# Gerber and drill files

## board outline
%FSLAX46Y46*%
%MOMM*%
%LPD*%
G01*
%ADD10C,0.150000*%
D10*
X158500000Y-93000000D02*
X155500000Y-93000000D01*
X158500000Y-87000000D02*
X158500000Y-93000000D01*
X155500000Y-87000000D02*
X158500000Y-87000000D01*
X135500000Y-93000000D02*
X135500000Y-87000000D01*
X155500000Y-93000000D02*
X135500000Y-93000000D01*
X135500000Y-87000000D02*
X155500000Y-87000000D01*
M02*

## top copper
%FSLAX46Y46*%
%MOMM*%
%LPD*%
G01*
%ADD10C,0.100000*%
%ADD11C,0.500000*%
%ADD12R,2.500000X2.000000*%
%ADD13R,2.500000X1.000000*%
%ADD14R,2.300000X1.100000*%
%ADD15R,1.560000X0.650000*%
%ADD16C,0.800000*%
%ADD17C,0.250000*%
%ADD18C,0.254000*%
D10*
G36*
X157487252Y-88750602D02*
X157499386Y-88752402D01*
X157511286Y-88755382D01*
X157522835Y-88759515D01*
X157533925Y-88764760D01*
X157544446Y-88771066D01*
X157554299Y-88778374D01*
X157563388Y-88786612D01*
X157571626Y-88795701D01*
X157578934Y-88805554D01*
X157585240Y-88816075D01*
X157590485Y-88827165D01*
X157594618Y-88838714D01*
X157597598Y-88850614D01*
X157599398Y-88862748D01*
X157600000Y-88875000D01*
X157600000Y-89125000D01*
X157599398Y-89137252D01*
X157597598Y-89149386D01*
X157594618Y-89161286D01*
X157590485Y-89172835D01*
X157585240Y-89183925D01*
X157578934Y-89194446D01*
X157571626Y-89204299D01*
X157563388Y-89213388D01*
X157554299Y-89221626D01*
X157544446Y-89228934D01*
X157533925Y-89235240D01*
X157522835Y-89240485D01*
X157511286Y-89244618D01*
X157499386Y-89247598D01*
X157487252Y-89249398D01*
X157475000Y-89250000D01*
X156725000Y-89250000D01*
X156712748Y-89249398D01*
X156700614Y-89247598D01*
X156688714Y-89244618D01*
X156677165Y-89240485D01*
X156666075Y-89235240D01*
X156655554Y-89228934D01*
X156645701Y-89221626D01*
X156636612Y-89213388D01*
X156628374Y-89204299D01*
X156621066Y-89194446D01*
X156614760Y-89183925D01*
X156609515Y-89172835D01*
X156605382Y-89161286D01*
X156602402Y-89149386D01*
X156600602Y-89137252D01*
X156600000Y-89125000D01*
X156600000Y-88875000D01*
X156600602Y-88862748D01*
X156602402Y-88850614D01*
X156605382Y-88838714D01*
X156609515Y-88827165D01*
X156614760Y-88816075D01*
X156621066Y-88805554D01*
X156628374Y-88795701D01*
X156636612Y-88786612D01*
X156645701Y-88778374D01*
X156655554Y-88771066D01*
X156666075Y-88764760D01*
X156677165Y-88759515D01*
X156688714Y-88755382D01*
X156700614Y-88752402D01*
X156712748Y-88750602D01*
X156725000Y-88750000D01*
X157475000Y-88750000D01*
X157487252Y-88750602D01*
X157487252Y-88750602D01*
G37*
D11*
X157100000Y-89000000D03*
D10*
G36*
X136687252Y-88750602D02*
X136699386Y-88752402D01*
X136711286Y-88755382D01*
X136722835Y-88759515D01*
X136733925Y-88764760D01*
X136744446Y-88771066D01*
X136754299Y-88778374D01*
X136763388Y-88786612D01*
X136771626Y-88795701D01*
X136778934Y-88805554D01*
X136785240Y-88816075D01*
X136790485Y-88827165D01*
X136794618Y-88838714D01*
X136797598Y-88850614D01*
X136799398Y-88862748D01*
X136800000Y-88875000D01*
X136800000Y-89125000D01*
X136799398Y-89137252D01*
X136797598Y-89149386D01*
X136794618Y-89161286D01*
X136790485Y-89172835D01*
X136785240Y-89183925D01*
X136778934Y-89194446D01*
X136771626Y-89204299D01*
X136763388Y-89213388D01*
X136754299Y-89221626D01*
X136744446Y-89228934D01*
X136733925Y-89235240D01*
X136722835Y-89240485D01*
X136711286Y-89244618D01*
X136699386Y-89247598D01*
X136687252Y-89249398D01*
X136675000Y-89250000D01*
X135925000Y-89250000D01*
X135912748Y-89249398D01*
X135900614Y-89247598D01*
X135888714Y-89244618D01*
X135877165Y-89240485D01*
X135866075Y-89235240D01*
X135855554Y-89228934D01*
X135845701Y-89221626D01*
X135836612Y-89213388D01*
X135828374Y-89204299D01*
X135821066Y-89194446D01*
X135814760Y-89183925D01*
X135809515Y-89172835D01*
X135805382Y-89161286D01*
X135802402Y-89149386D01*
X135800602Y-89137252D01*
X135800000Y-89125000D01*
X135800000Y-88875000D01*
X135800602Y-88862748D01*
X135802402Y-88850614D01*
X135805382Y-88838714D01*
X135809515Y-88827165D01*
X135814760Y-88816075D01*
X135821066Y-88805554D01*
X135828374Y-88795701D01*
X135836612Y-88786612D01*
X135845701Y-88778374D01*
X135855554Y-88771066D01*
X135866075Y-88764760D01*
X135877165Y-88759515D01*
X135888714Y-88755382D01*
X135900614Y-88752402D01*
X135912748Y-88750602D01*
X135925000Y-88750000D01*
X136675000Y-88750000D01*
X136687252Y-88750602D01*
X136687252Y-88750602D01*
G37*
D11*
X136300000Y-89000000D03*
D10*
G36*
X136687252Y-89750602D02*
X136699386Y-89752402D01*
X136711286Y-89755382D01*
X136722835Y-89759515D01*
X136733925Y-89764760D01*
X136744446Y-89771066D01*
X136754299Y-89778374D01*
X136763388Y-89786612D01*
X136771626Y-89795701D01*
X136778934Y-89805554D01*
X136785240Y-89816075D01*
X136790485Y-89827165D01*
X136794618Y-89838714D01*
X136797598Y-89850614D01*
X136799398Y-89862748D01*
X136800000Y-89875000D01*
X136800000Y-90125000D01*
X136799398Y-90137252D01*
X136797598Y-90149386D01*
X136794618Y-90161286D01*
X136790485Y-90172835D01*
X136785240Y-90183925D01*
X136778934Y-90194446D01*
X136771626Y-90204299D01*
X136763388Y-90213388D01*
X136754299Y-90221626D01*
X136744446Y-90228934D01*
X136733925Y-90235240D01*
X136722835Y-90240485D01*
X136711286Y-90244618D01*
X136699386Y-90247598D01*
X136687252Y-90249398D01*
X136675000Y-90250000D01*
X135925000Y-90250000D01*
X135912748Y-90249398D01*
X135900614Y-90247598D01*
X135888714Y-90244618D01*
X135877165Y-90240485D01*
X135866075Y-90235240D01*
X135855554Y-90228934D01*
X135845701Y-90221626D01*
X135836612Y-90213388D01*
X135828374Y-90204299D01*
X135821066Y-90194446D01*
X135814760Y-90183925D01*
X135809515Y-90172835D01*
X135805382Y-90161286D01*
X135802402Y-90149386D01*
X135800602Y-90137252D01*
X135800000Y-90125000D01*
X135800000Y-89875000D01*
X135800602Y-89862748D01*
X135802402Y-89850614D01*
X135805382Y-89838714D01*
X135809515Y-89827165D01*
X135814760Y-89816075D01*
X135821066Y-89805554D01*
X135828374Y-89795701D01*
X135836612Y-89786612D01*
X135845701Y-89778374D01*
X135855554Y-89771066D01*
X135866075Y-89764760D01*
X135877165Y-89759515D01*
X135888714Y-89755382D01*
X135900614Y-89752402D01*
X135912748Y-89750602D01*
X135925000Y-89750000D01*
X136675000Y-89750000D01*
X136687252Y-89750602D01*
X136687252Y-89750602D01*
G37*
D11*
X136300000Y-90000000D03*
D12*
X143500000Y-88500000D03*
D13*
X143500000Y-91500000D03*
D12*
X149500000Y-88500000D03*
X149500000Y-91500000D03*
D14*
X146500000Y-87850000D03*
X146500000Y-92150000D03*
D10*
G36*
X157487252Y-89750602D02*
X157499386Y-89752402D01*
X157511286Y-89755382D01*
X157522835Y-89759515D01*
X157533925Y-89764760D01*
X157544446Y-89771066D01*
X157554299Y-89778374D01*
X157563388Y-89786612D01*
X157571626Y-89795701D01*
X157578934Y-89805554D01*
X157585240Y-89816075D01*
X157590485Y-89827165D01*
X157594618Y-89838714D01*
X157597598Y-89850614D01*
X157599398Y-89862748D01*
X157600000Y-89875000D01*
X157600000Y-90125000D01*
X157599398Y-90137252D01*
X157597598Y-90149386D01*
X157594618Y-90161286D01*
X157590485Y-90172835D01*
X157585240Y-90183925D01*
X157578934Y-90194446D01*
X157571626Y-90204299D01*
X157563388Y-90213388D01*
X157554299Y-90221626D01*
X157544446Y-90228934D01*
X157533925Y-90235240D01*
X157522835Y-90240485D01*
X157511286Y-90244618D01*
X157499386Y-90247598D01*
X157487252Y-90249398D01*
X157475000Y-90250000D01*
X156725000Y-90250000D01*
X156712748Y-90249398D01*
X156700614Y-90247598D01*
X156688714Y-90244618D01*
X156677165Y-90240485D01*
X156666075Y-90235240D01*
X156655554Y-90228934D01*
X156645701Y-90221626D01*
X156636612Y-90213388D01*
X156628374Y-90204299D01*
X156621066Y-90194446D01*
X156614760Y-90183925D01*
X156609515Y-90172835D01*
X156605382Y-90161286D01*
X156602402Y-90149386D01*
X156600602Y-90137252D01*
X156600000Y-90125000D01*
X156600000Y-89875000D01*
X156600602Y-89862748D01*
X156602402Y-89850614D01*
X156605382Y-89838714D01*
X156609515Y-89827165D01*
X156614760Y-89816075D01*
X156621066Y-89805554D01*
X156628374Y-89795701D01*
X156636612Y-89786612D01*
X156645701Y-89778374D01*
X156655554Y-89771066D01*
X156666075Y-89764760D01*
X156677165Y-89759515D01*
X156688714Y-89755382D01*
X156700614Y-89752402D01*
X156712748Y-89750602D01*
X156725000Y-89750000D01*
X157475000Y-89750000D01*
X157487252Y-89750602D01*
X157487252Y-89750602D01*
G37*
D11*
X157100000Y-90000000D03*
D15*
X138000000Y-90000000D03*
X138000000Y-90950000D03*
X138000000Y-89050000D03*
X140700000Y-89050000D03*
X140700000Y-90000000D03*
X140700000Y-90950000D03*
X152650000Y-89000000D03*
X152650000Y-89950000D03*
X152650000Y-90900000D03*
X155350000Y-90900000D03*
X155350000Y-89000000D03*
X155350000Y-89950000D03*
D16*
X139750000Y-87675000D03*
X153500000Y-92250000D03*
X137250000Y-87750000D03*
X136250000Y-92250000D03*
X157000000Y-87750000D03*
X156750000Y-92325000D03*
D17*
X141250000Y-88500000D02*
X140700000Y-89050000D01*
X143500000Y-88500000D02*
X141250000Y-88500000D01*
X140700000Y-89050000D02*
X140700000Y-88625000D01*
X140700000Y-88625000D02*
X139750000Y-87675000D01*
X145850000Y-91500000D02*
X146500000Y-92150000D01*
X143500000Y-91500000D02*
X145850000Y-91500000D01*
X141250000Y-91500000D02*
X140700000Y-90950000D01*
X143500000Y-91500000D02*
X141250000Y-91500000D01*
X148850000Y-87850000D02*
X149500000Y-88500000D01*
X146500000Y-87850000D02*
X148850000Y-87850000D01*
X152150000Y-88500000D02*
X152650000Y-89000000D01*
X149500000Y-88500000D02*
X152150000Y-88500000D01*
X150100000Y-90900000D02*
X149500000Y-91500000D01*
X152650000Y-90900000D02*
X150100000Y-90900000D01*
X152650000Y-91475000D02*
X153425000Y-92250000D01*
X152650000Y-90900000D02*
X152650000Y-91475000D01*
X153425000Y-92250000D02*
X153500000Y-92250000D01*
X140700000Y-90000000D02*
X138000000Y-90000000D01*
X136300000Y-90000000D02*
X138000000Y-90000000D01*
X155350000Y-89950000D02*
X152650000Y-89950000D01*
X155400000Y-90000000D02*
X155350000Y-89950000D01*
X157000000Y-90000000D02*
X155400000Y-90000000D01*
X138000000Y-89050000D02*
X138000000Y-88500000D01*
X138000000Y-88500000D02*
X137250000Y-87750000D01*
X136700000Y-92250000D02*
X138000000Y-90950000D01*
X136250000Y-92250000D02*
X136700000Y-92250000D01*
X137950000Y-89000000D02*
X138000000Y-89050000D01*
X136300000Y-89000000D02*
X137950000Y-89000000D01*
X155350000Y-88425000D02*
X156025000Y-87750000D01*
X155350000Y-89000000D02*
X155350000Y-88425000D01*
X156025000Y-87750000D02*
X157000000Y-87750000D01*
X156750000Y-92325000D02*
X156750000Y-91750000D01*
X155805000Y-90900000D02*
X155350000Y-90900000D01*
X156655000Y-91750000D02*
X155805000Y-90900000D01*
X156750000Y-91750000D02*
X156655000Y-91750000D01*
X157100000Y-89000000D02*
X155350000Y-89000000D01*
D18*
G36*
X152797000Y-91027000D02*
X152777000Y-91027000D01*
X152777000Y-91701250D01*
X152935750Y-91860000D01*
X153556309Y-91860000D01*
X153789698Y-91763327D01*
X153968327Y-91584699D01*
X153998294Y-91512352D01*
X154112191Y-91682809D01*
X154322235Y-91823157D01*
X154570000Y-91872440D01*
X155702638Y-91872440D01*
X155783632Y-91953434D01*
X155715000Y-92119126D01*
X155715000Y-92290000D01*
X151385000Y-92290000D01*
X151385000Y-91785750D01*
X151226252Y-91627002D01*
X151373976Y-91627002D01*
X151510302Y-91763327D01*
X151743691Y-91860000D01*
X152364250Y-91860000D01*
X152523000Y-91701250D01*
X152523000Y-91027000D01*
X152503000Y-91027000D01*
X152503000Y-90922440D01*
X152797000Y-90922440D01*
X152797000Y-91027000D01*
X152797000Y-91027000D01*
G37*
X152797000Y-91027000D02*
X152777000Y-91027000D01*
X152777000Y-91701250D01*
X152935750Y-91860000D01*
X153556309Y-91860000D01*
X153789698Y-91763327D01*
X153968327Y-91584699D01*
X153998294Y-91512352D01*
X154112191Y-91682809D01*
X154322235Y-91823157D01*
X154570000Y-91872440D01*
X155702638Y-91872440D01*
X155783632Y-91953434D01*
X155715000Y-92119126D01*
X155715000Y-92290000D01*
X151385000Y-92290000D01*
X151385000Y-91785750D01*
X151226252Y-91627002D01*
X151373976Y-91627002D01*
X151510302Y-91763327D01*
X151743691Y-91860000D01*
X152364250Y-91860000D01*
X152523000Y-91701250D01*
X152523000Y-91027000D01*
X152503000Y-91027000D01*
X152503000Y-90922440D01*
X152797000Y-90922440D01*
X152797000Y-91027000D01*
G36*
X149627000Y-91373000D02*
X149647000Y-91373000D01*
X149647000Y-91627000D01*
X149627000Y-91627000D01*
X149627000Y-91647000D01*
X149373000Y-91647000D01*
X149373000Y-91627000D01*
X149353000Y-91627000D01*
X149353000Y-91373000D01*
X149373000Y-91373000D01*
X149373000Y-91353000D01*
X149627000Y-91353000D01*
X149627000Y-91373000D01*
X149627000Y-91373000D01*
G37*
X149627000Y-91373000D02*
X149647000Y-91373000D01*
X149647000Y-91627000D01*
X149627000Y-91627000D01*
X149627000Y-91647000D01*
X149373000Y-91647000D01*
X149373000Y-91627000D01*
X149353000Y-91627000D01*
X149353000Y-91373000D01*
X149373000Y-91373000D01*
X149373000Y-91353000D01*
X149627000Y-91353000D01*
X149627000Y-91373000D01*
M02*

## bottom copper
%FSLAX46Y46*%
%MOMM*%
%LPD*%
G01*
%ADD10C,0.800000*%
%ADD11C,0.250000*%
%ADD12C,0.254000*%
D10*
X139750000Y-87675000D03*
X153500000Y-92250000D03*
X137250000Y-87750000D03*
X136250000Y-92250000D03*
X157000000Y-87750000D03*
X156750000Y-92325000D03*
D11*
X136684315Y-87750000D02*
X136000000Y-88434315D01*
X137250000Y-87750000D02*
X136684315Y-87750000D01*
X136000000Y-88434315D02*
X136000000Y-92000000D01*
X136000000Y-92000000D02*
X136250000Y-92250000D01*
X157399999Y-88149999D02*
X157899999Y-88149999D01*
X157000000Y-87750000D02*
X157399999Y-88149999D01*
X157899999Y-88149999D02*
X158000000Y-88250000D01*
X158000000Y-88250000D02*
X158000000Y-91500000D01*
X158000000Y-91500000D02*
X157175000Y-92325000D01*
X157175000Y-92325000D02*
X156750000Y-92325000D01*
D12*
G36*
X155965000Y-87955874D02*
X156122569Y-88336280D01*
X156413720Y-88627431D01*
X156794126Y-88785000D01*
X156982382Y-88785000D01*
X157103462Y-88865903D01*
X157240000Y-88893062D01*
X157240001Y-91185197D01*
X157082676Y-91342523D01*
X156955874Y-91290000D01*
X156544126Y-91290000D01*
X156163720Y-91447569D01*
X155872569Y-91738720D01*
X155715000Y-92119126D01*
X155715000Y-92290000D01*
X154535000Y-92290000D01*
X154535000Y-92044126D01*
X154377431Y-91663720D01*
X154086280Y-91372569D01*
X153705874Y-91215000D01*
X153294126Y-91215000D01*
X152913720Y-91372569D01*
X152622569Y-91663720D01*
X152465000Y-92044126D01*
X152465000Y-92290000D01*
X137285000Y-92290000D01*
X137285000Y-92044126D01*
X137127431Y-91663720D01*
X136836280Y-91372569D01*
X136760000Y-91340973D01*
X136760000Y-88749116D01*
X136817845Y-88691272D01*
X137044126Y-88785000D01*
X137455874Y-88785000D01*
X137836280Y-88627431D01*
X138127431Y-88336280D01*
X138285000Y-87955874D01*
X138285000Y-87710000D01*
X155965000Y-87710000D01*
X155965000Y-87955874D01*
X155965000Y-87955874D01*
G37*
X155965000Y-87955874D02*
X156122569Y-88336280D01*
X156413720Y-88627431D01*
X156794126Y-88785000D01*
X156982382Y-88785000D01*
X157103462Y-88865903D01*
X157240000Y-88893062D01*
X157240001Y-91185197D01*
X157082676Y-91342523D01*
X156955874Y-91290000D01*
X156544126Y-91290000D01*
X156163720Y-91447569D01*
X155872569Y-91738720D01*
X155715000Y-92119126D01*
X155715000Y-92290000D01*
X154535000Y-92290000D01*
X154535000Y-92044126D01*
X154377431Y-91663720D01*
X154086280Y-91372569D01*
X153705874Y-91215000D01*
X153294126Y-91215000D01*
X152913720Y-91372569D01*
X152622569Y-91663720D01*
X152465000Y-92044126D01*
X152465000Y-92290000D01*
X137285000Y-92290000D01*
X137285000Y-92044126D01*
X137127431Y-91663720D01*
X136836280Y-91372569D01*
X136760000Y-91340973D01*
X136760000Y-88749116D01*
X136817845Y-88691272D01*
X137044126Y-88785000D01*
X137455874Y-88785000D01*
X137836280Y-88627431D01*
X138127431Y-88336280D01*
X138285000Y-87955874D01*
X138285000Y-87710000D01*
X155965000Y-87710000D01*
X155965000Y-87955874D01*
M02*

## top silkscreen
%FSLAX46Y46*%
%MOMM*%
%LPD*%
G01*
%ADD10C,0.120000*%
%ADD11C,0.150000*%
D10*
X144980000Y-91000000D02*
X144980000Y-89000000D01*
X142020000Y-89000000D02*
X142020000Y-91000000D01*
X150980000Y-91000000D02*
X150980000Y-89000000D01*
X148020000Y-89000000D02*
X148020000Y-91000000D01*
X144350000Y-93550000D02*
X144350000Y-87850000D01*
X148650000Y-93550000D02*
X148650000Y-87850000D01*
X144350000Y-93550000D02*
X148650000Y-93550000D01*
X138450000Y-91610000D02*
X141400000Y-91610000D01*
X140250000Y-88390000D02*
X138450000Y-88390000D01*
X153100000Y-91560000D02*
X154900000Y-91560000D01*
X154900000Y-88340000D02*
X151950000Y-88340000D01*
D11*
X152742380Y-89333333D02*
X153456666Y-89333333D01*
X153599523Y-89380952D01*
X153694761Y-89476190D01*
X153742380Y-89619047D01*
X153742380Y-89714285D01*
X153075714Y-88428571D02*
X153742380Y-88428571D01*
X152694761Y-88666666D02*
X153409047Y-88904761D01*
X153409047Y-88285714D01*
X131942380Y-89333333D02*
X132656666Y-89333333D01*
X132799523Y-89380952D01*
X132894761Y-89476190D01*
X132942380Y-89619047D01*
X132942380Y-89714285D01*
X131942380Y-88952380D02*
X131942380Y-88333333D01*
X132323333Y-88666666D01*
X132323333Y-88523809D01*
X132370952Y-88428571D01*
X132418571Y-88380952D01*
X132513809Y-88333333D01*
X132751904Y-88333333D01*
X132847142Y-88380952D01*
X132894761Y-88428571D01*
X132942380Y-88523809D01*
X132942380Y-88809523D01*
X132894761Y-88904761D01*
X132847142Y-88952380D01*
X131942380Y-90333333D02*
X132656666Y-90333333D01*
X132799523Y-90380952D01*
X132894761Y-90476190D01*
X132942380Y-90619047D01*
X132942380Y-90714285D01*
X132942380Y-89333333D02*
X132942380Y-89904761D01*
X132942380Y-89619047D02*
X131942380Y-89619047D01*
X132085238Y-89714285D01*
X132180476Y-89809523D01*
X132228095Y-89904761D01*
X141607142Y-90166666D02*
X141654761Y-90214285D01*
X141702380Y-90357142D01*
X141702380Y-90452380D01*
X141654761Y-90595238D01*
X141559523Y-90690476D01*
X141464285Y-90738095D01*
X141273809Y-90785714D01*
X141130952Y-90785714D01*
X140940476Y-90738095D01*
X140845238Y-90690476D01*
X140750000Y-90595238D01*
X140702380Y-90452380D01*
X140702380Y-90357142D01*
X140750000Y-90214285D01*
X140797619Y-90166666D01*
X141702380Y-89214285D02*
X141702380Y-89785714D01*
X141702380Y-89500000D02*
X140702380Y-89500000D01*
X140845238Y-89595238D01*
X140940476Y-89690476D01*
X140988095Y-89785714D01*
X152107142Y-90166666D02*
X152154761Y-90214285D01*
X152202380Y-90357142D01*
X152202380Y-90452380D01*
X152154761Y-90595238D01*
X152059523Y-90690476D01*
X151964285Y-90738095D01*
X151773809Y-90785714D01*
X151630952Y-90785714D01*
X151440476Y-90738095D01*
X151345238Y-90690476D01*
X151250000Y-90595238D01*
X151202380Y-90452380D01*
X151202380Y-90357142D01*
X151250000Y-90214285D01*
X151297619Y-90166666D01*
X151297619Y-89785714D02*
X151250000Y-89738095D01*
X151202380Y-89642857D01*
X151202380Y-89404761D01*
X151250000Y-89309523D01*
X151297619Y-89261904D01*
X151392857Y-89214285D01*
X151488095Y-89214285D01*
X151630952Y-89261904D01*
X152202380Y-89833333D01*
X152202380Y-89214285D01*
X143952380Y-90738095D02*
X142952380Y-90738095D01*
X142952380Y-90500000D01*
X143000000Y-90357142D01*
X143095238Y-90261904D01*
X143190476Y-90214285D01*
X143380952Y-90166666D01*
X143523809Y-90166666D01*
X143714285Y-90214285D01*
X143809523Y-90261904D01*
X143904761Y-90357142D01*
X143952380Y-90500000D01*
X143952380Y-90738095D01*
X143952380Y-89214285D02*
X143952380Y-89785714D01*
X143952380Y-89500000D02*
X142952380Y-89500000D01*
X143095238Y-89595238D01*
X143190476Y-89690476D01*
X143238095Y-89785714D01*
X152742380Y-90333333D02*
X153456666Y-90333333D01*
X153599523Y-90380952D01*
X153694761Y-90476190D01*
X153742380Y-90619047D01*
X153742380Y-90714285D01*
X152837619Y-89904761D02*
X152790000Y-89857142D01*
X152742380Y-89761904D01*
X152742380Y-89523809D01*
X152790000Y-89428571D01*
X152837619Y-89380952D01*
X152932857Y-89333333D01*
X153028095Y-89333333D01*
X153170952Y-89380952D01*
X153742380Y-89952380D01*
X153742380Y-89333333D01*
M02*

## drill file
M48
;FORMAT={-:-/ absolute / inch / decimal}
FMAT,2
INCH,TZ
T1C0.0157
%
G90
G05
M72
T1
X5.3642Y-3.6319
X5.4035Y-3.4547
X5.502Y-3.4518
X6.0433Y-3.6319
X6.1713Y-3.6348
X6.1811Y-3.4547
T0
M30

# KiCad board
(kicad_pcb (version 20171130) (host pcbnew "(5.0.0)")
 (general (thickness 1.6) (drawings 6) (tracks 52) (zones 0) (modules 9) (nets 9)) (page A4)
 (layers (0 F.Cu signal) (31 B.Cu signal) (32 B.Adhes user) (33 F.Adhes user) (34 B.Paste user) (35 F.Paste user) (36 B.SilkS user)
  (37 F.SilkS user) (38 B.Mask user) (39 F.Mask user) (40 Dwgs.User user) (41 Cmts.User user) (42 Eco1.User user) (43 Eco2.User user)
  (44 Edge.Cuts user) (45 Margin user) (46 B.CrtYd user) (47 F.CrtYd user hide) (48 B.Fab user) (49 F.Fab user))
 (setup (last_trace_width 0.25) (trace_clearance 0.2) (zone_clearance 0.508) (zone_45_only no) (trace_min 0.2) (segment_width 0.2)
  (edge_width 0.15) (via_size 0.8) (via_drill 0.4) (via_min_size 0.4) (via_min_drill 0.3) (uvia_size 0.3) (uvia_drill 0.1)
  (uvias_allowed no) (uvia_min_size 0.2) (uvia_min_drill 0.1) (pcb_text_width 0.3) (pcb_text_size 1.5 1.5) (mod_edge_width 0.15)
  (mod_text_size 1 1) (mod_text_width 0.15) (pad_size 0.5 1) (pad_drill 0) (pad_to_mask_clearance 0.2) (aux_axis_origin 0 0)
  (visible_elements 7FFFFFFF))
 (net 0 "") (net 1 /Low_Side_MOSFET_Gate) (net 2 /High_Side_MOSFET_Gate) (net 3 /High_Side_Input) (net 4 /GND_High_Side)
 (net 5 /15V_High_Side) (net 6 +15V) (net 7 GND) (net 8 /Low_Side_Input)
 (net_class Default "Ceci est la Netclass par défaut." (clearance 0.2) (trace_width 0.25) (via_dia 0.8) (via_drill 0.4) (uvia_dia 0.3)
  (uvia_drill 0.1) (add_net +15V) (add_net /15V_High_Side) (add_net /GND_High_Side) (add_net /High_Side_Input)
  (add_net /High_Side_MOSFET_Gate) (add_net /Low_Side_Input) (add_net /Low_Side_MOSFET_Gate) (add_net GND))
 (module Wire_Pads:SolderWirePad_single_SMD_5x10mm (layer F.Cu) (at 157.1 89 90)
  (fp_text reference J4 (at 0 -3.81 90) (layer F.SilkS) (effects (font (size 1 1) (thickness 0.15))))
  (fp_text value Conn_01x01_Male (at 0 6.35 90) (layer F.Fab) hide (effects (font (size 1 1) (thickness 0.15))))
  (pad 1 smd roundrect (at 0 0 90) (size 0.5 1) (layers F.Cu F.Paste F.Mask) (roundrect_rratio 0.25) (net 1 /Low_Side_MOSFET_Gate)))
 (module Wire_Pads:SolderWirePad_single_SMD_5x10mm (layer F.Cu) (at 136.3 89 90)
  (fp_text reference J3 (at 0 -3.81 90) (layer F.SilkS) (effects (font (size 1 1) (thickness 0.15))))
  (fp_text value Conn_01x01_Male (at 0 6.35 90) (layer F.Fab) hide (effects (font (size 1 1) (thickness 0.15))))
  (pad 1 smd roundrect (at 0 0 90) (size 0.5 1) (layers F.Cu F.Paste F.Mask) (roundrect_rratio 0.25) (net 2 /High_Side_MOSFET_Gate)))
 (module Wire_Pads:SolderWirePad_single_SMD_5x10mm (layer F.Cu) (at 136.3 90 90)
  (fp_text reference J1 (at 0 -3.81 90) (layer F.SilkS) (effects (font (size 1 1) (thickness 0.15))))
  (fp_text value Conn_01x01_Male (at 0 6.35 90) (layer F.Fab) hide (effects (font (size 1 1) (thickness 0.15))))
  (pad 1 smd roundrect (at 0 0 90) (size 0.5 1) (layers F.Cu F.Paste F.Mask) (roundrect_rratio 0.25) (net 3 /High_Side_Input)))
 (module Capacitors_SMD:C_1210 (layer F.Cu) (at 143.5 90 90)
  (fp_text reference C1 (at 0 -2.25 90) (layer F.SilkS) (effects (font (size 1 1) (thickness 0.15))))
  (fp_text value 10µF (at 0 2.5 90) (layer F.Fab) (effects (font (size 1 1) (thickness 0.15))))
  (fp_line (start -1 1.48) (end 1 1.48) (layer F.SilkS) (width 0.12))
  (fp_line (start 1 -1.48) (end -1 -1.48) (layer F.SilkS) (width 0.12))
  (pad 2 smd rect (at 1.5 0 90) (size 2 2.5) (layers F.Cu F.Paste F.Mask) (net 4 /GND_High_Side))
  (pad 1 smd rect (at -1.5 0 90) (size 1 2.5) (layers F.Cu F.Paste F.Mask) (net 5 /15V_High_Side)))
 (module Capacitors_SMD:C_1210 (layer F.Cu) (at 149.5 90 270)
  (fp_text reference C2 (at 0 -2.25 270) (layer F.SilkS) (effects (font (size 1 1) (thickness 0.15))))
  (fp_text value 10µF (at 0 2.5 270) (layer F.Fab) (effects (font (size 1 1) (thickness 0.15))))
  (fp_line (start 1 -1.48) (end -1 -1.48) (layer F.SilkS) (width 0.12))
  (fp_line (start -1 1.48) (end 1 1.48) (layer F.SilkS) (width 0.12))
  (pad 1 smd rect (at -1.5 0 270) (size 2 2.5) (layers F.Cu F.Paste F.Mask) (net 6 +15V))
  (pad 2 smd rect (at 1.5 0 270) (size 2 2.5) (layers F.Cu F.Paste F.Mask) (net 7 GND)))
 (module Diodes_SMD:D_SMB (layer F.Cu) (at 146.5 90 90)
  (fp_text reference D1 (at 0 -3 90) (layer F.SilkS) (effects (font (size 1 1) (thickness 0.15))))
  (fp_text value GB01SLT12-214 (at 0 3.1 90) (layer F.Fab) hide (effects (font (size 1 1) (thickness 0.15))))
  (fp_line (start -3.55 -2.15) (end 2.15 -2.15) (layer F.SilkS) (width 0.12))
  (fp_line (start -3.55 2.15) (end 2.15 2.15) (layer F.SilkS) (width 0.12))
  (fp_line (start -3.55 -2.15) (end -3.55 2.15) (layer F.SilkS) (width 0.12))
  (pad 2 smd rect (at 2.15 0 90) (size 1.1 2.3) (layers F.Cu F.Paste F.Mask) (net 6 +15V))
  (pad 1 smd rect (at -2.15 0 90) (size 1.1 2.3) (layers F.Cu F.Paste F.Mask) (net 5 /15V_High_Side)))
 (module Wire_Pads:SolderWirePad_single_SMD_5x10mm (layer F.Cu) (at 157.1 90 90)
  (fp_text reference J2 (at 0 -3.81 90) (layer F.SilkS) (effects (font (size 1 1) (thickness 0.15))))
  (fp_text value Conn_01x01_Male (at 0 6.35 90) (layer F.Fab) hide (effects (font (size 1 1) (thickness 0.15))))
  (pad 1 smd roundrect (at 0 0 90) (size 0.5 1) (layers F.Cu F.Paste F.Mask) (roundrect_rratio 0.25) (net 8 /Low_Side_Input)
   (zone_connect 0)))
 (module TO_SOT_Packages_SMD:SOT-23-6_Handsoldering (layer F.Cu) (at 139.35 90 180)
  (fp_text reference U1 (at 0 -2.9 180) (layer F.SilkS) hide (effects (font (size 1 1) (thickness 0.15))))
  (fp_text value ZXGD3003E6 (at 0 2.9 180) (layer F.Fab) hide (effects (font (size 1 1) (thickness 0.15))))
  (fp_line (start 0.9 -1.61) (end -2.05 -1.61) (layer F.SilkS) (width 0.12))
  (fp_line (start -0.9 1.61) (end 0.9 1.61) (layer F.SilkS) (width 0.12))
  (pad 5 smd rect (at 1.35 0 180) (size 1.56 0.65) (layers F.Cu F.Paste F.Mask) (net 3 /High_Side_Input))
  (pad 6 smd rect (at 1.35 -0.95 180) (size 1.56 0.65) (layers F.Cu F.Paste F.Mask) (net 2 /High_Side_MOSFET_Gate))
  (pad 4 smd rect (at 1.35 0.95 180) (size 1.56 0.65) (layers F.Cu F.Paste F.Mask) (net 2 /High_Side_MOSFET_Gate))
  (pad 3 smd rect (at -1.35 0.95 180) (size 1.56 0.65) (layers F.Cu F.Paste F.Mask) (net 4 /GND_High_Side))
  (pad 2 smd rect (at -1.35 0 180) (size 1.56 0.65) (layers F.Cu F.Paste F.Mask) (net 3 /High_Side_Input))
  (pad 1 smd rect (at -1.35 -0.95 180) (size 1.56 0.65) (layers F.Cu F.Paste F.Mask) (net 5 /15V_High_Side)))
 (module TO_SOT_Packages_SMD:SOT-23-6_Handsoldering (layer F.Cu) (at 154 89.95)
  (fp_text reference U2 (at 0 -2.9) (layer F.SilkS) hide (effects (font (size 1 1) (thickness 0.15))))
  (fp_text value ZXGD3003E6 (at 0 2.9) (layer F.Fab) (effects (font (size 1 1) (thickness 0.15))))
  (fp_line (start -0.9 1.61) (end 0.9 1.61) (layer F.SilkS) (width 0.12))
  (fp_line (start 0.9 -1.61) (end -2.05 -1.61) (layer F.SilkS) (width 0.12))
  (pad 1 smd rect (at -1.35 -0.95) (size 1.56 0.65) (layers F.Cu F.Paste F.Mask) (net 6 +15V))
  (pad 2 smd rect (at -1.35 0) (size 1.56 0.65) (layers F.Cu F.Paste F.Mask) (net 8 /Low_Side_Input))
  (pad 3 smd rect (at -1.35 0.95) (size 1.56 0.65) (layers F.Cu F.Paste F.Mask) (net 7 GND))
  (pad 4 smd rect (at 1.35 0.95) (size 1.56 0.65) (layers F.Cu F.Paste F.Mask) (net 1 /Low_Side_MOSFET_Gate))
  (pad 6 smd rect (at 1.35 -0.95) (size 1.56 0.65) (layers F.Cu F.Paste F.Mask) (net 1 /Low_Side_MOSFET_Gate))
  (pad 5 smd rect (at 1.35 0) (size 1.56 0.65) (layers F.Cu F.Paste F.Mask) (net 8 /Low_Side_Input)))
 (gr_line (start 158.5 93) (end 155.5 93) (layer Edge.Cuts) (width 0.15))
 (gr_line (start 158.5 87) (end 158.5 93) (layer Edge.Cuts) (width 0.15))
 (gr_line (start 155.5 87) (end 158.5 87) (layer Edge.Cuts) (width 0.15))
 (gr_line (start 135.5 93) (end 135.5 87) (layer Edge.Cuts) (width 0.15))
 (gr_line (start 155.5 93) (end 135.5 93) (layer Edge.Cuts) (width 0.15))
 (gr_line (start 135.5 87) (end 155.5 87) (layer Edge.Cuts) (width 0.15))
 (segment (start 141.25 88.5) (end 140.7 89.05) (width 0.25) (layer F.Cu) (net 4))
 (segment (start 143.5 88.5) (end 141.25 88.5) (width 0.25) (layer F.Cu) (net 4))
 (via (at 139.75 87.675) (size 0.8) (drill 0.4) (layers F.Cu B.Cu) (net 4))
 (segment (start 140.7 89.05) (end 140.7 88.625) (width 0.25) (layer F.Cu) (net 4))
 (segment (start 140.7 88.625) (end 139.75 87.675) (width 0.25) (layer F.Cu) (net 4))
 (segment (start 145.85 91.5) (end 146.5 92.15) (width 0.25) (layer F.Cu) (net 5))
 (segment (start 143.5 91.5) (end 145.85 91.5) (width 0.25) (layer F.Cu) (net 5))
 (segment (start 141.25 91.5) (end 140.7 90.95) (width 0.25) (layer F.Cu) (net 5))
 (segment (start 143.5 91.5) (end 141.25 91.5) (width 0.25) (layer F.Cu) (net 5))
 (segment (start 148.85 87.85) (end 149.5 88.5) (width 0.25) (layer F.Cu) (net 6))
 (segment (start 146.5 87.85) (end 148.85 87.85) (width 0.25) (layer F.Cu) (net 6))
 (segment (start 152.15 88.5) (end 152.65 89) (width 0.25) (layer F.Cu) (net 6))
 (segment (start 149.5 88.5) (end 152.15 88.5) (width 0.25) (layer F.Cu) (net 6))
 (segment (start 150.1 90.9) (end 149.5 91.5) (width 0.25) (layer F.Cu) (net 7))
 (segment (start 152.65 90.9) (end 150.1 90.9) (width 0.25) (layer F.Cu) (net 7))
 (segment (start 152.65 91.475) (end 153.425 92.25) (width 0.25) (layer F.Cu) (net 7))
 (segment (start 152.65 90.9) (end 152.65 91.475) (width 0.25) (layer F.Cu) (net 7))
 (via (at 153.5 92.25) (size 0.8) (drill 0.4) (layers F.Cu B.Cu) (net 7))
 (segment (start 153.425 92.25) (end 153.5 92.25) (width 0.25) (layer F.Cu) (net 7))
 (segment (start 140.7 90) (end 138 90) (width 0.25) (layer F.Cu) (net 3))
 (segment (start 136.3 90) (end 138 90) (width 0.25) (layer F.Cu) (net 3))
 (segment (start 155.35 89.95) (end 152.65 89.95) (width 0.25) (layer F.Cu) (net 8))
 (segment (start 155.4 90) (end 155.35 89.95) (width 0.25) (layer F.Cu) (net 8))
 (segment (start 157 90) (end 155.4 90) (width 0.25) (layer F.Cu) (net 8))
 (via (at 137.25 87.75) (size 0.8) (drill 0.4) (layers F.Cu B.Cu) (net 2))
 (segment (start 138 89.05) (end 138 88.5) (width 0.25) (layer F.Cu) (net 2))
 (segment (start 138 88.5) (end 137.25 87.75) (width 0.25) (layer F.Cu) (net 2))
 (segment (start 136.684315 87.75) (end 136 88.434315) (width 0.25) (layer B.Cu) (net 2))
 (segment (start 137.25 87.75) (end 136.684315 87.75) (width 0.25) (layer B.Cu) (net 2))
 (via (at 136.25 92.25) (size 0.8) (drill 0.4) (layers F.Cu B.Cu) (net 2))
 (segment (start 136 88.434315) (end 136 92) (width 0.25) (layer B.Cu) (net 2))
 (segment (start 136 92) (end 136.25 92.25) (width 0.25) (layer B.Cu) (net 2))
 (segment (start 136.7 92.25) (end 138 90.95) (width 0.25) (layer F.Cu) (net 2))
 (segment (start 136.25 92.25) (end 136.7 92.25) (width 0.25) (layer F.Cu) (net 2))
 (segment (start 137.95 89) (end 138 89.05) (width 0.25) (layer F.Cu) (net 2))
 (segment (start 136.3 89) (end 137.95 89) (width 0.25) (layer F.Cu) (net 2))
 (segment (start 155.35 88.425) (end 156.025 87.75) (width 0.25) (layer F.Cu) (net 1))
 (segment (start 155.35 89) (end 155.35 88.425) (width 0.25) (layer F.Cu) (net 1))
 (via (at 157 87.75) (size 0.8) (drill 0.4) (layers F.Cu B.Cu) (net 1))
 (segment (start 156.025 87.75) (end 157 87.75) (width 0.25) (layer F.Cu) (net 1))
 (segment (start 157.399999 88.149999) (end 157.899999 88.149999) (width 0.25) (layer B.Cu) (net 1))
 (segment (start 157 87.75) (end 157.399999 88.149999) (width 0.25) (layer B.Cu) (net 1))
 (segment (start 157.899999 88.149999) (end 158 88.25) (width 0.25) (layer B.Cu) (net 1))
 (segment (start 158 88.25) (end 158 91.5) (width 0.25) (layer B.Cu) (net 1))
 (via (at 156.75 92.325) (size 0.8) (drill 0.4) (layers F.Cu B.Cu) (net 1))
 (segment (start 158 91.5) (end 157.175 92.325) (width 0.25) (layer B.Cu) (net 1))
 (segment (start 157.175 92.325) (end 156.75 92.325) (width 0.25) (layer B.Cu) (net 1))
 (segment (start 156.75 92.325) (end 156.75 91.75) (width 0.25) (layer F.Cu) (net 1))
 (segment (start 155.805 90.9) (end 155.35 90.9) (width 0.25) (layer F.Cu) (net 1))
 (segment (start 156.655 91.75) (end 155.805 90.9) (width 0.25) (layer F.Cu) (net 1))
 (segment (start 156.75 91.75) (end 156.655 91.75) (width 0.25) (layer F.Cu) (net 1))
 (segment (start 157.1 89) (end 155.35 89) (width 0.25) (layer F.Cu) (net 1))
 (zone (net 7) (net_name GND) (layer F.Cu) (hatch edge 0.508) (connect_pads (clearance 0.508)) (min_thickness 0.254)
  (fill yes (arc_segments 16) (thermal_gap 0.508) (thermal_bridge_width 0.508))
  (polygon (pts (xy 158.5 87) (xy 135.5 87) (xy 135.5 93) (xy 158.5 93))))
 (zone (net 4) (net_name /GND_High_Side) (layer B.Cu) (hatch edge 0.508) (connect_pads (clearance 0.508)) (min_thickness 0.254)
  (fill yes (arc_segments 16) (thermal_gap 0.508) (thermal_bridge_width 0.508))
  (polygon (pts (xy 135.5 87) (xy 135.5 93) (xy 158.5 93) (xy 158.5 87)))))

